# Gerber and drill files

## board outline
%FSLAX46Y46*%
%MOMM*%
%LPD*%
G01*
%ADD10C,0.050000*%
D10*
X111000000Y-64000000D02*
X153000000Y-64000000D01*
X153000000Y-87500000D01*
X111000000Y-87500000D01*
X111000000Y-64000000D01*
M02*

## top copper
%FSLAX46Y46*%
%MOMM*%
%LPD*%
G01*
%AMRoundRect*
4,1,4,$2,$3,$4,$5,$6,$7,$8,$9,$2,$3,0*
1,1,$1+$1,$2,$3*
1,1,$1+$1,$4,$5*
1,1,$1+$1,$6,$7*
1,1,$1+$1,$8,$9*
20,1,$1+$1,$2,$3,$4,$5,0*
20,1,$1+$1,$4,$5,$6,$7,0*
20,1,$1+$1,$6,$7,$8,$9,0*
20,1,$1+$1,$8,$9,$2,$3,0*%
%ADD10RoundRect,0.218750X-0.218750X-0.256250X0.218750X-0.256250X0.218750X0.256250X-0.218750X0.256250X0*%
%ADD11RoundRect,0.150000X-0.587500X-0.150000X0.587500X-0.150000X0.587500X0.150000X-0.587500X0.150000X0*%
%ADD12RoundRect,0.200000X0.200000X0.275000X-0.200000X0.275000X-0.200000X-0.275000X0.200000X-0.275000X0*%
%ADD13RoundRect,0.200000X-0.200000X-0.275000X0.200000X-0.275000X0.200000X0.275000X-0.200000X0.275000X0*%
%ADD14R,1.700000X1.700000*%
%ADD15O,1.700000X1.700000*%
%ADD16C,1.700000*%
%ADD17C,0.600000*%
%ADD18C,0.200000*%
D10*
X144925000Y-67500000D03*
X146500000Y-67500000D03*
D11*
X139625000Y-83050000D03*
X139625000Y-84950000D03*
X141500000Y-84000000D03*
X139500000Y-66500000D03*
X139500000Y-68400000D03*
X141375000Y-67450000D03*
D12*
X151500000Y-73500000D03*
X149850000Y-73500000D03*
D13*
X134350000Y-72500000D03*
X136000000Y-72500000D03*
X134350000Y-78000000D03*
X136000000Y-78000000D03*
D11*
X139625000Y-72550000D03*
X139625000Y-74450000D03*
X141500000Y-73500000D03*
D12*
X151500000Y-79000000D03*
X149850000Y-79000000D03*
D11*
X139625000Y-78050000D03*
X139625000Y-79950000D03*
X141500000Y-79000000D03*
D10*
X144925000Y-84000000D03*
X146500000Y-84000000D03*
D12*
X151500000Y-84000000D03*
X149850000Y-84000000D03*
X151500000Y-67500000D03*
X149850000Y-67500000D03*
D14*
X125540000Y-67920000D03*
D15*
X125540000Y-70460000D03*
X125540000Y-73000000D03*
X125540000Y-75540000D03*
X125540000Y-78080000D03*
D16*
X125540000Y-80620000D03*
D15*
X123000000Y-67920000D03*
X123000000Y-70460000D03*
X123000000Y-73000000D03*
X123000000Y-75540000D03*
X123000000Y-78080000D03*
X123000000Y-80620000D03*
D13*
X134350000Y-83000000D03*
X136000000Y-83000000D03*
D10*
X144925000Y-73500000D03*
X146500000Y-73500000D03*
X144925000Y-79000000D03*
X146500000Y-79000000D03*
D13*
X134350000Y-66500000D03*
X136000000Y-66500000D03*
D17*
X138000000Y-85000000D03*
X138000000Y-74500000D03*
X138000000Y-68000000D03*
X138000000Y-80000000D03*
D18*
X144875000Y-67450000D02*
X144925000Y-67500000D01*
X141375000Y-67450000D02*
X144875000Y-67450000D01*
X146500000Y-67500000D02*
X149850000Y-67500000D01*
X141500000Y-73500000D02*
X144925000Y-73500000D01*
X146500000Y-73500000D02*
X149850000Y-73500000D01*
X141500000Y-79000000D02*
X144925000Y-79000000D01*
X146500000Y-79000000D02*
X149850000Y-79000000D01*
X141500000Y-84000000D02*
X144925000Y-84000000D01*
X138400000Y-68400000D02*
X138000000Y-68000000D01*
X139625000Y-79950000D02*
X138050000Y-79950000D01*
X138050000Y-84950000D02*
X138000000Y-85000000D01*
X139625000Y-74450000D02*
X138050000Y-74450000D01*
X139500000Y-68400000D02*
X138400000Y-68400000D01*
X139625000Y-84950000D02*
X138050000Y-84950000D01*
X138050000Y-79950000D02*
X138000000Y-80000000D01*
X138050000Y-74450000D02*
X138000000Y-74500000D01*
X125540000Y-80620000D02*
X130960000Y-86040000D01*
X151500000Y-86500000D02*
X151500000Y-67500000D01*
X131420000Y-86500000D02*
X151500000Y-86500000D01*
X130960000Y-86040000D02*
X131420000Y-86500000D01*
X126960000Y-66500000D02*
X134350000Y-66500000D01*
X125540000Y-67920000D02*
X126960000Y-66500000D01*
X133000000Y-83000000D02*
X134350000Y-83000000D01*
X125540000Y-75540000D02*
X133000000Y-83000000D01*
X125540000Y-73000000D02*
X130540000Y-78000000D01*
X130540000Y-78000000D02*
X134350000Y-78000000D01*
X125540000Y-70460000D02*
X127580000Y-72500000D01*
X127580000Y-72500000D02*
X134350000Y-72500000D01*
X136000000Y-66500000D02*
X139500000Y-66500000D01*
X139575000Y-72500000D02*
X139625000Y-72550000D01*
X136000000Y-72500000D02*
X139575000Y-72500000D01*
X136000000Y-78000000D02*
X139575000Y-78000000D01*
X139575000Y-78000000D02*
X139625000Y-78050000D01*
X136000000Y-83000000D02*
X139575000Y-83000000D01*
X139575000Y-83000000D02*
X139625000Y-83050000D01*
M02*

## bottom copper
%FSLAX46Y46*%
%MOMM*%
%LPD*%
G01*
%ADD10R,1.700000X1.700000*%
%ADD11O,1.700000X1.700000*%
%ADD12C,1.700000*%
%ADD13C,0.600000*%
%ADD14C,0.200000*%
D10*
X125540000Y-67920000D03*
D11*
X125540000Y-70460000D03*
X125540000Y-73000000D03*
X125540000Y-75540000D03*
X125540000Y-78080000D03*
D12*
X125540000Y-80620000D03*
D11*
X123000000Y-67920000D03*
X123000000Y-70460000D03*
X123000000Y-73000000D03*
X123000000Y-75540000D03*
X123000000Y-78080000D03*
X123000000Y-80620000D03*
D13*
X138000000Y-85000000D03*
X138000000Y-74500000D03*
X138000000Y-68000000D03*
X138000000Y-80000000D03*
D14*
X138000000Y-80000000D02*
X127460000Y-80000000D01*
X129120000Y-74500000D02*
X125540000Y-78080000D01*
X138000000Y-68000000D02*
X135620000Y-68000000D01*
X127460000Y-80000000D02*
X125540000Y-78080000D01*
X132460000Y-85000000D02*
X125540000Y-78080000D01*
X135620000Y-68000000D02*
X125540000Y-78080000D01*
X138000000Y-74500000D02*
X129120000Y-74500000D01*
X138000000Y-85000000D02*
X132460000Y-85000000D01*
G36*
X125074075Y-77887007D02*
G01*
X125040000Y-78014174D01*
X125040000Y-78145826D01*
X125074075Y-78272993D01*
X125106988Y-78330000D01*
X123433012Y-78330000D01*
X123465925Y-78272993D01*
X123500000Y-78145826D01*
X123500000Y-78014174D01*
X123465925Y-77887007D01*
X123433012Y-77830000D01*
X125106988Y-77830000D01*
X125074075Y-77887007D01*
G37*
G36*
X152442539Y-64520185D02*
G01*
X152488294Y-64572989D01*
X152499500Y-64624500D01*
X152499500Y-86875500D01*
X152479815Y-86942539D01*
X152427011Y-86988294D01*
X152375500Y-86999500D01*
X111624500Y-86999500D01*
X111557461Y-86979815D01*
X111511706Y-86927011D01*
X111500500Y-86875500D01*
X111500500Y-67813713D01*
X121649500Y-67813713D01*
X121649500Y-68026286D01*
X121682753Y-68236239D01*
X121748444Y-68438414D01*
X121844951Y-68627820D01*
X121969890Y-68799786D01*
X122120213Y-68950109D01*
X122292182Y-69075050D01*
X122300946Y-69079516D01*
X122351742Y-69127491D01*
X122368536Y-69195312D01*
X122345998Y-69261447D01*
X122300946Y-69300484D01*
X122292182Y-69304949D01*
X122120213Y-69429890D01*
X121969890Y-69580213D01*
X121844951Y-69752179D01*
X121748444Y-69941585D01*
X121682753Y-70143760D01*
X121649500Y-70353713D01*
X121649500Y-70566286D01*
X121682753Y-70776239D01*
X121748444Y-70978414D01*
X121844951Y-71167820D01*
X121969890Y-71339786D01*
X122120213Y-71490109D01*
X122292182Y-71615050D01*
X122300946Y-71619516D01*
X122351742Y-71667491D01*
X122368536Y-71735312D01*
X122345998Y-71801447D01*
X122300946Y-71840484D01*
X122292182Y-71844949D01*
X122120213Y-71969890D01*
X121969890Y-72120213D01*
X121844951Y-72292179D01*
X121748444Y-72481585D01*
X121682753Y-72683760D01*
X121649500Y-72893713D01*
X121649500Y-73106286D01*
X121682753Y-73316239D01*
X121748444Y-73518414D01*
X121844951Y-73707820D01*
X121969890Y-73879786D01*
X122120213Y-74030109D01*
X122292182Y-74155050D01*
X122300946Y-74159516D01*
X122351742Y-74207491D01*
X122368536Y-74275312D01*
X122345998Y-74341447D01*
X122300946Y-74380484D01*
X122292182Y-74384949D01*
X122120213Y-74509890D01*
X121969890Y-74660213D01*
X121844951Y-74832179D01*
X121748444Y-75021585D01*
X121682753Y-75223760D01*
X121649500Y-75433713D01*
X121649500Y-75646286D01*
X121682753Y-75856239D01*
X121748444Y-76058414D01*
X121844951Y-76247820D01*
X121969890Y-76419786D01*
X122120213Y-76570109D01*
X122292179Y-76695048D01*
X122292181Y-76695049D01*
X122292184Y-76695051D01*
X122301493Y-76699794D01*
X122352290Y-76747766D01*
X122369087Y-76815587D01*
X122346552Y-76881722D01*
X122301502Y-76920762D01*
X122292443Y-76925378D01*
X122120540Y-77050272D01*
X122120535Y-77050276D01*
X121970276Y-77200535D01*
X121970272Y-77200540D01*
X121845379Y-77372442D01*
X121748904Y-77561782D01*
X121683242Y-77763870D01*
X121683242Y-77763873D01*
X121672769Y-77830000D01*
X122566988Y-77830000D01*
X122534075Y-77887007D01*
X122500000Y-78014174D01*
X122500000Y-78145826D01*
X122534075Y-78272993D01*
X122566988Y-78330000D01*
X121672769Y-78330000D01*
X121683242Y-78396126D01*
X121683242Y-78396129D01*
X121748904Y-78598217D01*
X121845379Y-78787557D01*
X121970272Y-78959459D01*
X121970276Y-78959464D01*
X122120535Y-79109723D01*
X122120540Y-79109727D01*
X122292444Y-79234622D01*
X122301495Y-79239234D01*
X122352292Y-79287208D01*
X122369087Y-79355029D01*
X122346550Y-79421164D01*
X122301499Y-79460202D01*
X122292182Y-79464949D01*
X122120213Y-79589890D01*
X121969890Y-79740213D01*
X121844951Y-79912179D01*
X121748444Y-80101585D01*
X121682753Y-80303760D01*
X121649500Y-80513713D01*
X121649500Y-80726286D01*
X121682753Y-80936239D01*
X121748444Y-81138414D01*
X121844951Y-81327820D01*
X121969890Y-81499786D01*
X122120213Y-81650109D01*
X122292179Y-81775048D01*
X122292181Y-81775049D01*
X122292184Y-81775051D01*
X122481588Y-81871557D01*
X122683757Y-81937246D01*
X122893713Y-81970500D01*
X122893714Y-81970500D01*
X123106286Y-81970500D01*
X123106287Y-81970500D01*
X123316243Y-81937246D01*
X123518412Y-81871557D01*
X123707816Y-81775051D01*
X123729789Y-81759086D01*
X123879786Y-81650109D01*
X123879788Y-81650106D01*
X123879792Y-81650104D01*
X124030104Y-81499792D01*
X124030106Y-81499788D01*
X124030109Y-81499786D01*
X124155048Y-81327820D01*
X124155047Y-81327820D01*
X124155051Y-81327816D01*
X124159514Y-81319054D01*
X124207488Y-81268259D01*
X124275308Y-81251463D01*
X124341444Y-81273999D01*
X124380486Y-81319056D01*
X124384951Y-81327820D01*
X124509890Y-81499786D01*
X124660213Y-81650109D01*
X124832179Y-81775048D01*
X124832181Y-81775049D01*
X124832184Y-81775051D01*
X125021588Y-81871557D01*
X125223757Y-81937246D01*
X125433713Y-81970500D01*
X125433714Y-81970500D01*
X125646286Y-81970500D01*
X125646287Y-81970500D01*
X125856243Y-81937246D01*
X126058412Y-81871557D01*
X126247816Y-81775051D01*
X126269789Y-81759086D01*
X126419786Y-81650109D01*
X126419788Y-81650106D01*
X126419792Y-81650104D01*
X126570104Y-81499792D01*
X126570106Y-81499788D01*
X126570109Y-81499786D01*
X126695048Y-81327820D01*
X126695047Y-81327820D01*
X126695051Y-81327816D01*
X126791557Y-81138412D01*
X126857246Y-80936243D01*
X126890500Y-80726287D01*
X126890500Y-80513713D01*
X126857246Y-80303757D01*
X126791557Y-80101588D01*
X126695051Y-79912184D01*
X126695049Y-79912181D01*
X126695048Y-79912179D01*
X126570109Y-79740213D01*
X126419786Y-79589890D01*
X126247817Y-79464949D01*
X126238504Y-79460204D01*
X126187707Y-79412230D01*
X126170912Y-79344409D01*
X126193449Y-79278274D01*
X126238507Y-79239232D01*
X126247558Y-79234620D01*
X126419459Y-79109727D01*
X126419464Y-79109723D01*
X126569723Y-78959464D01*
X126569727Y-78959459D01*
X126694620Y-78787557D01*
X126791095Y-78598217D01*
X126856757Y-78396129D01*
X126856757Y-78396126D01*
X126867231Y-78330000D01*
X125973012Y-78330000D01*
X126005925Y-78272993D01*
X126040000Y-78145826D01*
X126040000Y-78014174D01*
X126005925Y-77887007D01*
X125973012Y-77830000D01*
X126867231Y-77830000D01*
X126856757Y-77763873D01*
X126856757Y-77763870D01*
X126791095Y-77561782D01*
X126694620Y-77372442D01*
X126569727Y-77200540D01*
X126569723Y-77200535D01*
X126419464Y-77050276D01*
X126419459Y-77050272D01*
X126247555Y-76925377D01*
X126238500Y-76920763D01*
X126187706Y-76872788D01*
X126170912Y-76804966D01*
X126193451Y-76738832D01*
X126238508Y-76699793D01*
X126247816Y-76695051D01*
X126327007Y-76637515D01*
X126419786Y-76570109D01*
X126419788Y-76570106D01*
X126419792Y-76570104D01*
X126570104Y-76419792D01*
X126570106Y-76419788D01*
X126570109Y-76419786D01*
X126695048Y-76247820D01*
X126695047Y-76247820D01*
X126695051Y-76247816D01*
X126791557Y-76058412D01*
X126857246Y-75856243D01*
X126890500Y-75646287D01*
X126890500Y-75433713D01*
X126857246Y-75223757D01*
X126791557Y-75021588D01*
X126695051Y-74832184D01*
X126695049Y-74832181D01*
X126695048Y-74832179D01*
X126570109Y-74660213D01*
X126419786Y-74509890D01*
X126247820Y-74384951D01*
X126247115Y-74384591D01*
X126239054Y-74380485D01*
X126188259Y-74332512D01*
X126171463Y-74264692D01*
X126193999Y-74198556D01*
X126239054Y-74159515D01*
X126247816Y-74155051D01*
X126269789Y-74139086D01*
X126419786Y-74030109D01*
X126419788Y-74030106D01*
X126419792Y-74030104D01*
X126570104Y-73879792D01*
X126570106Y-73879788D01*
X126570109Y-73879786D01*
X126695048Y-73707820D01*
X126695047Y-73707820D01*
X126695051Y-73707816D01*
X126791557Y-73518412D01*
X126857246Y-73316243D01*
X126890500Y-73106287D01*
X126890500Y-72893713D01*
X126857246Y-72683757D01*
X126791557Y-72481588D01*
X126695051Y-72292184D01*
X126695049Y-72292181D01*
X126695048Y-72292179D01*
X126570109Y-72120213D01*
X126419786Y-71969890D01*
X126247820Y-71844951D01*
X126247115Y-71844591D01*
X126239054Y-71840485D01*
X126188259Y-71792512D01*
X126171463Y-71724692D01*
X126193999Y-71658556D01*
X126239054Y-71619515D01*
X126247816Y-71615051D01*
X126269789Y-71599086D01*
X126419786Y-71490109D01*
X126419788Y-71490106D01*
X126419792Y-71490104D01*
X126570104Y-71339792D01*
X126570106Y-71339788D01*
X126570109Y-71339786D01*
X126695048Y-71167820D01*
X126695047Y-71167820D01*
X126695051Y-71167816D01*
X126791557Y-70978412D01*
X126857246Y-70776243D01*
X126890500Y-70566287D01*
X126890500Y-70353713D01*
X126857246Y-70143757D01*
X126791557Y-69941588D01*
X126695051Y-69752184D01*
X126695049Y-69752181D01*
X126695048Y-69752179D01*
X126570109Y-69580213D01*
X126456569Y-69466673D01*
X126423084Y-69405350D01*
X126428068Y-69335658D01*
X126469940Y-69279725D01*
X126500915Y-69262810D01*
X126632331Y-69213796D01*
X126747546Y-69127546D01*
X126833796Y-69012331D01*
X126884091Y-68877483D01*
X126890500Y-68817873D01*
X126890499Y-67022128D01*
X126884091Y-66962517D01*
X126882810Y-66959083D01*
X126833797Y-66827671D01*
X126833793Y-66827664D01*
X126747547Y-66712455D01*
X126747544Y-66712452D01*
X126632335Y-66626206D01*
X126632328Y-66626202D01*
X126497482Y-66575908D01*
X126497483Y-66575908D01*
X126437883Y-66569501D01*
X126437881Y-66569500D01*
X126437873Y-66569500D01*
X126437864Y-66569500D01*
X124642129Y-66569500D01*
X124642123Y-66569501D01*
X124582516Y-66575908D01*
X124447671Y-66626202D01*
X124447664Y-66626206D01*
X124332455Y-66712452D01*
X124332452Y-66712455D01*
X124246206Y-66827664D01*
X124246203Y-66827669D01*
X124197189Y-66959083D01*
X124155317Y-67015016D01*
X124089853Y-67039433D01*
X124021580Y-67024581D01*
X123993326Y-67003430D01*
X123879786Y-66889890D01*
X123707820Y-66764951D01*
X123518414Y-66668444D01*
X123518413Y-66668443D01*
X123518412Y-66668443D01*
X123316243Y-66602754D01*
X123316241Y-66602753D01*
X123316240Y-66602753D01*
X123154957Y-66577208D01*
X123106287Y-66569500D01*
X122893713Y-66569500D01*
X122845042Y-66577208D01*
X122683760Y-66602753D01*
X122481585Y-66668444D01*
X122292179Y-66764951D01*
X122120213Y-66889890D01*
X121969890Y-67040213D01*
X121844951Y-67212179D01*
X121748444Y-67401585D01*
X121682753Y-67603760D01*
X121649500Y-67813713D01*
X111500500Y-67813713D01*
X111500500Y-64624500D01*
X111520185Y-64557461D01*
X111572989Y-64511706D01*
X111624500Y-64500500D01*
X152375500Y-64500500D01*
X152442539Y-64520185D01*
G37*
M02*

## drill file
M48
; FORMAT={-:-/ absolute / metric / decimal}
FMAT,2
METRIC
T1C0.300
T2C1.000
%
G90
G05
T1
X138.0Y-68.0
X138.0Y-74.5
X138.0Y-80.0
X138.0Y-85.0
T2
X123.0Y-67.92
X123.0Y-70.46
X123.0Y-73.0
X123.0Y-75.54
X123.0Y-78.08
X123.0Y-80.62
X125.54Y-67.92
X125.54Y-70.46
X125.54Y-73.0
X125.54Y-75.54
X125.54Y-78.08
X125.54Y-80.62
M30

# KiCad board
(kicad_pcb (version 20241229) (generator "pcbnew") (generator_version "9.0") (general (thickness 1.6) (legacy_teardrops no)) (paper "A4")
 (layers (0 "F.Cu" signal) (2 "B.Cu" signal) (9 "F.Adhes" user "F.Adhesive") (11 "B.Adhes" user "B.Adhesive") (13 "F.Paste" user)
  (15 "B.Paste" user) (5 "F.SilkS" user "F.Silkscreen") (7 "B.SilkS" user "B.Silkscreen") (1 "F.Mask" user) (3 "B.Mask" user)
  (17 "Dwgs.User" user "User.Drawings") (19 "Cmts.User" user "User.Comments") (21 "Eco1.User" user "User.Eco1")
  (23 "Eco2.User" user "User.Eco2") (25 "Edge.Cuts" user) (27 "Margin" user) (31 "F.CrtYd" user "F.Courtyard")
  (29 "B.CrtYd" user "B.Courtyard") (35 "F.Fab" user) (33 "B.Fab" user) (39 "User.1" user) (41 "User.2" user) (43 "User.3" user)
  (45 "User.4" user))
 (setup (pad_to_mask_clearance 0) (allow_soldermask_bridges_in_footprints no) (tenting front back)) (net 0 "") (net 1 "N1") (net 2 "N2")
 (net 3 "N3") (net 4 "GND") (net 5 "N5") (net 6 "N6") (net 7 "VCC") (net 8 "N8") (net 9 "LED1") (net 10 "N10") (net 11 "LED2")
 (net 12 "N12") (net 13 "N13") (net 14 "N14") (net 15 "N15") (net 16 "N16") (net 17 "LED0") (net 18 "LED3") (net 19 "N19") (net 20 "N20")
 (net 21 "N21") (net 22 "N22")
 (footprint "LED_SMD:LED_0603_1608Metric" (layer "F.Cu") (at 145.7125 67.5)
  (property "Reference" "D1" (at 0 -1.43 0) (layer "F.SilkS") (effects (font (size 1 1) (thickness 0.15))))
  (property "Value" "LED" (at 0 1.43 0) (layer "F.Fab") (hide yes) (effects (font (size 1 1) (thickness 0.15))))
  (pad "1" smd roundrect (at -0.7875 0) (size 0.875 0.95) (layers "F.Cu" "F.Mask" "F.Paste") (roundrect_rratio 0.25) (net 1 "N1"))
  (pad "2" smd roundrect (at 0.7875 0) (size 0.875 0.95) (layers "F.Cu" "F.Mask" "F.Paste") (roundrect_rratio 0.25) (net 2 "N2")))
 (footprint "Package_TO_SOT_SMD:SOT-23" (layer "F.Cu") (at 140.5625 84)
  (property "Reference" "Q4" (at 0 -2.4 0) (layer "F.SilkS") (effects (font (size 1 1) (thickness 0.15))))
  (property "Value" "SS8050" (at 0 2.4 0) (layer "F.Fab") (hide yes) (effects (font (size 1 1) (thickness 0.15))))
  (pad "1" smd roundrect (at -0.9375 -0.95) (size 1.475 0.6) (layers "F.Cu" "F.Mask" "F.Paste") (roundrect_rratio 0.25) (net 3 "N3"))
  (pad "2" smd roundrect (at -0.9375 0.95) (size 1.475 0.6) (layers "F.Cu" "F.Mask" "F.Paste") (roundrect_rratio 0.25) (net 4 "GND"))
  (pad "3" smd roundrect (at 0.9375 0) (size 1.475 0.6) (layers "F.Cu" "F.Mask" "F.Paste") (roundrect_rratio 0.25) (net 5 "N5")))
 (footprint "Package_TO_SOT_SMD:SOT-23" (layer "F.Cu") (at 140.4375 67.45)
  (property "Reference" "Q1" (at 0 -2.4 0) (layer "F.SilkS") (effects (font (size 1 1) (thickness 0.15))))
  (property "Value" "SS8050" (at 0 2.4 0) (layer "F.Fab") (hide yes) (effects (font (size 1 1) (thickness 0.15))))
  (pad "1" smd roundrect (at -0.9375 -0.95) (size 1.475 0.6) (layers "F.Cu" "F.Mask" "F.Paste") (roundrect_rratio 0.25) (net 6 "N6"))
  (pad "2" smd roundrect (at -0.9375 0.95) (size 1.475 0.6) (layers "F.Cu" "F.Mask" "F.Paste") (roundrect_rratio 0.25) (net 4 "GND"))
  (pad "3" smd roundrect (at 0.9375 0) (size 1.475 0.6) (layers "F.Cu" "F.Mask" "F.Paste") (roundrect_rratio 0.25) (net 1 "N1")))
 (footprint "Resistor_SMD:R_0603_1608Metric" (layer "F.Cu") (at 150.675 73.5 180)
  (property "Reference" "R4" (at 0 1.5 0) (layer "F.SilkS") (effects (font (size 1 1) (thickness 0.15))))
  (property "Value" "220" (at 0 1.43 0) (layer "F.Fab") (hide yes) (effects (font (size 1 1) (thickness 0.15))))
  (pad "1" smd roundrect (at -0.825 0 180) (size 0.8 0.95) (layers "F.Cu" "F.Mask" "F.Paste") (roundrect_rratio 0.25) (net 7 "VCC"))
  (pad "2" smd roundrect (at 0.825 0 180) (size 0.8 0.95) (layers "F.Cu" "F.Mask" "F.Paste") (roundrect_rratio 0.25) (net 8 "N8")))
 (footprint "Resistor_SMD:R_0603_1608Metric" (layer "F.Cu") (at 135.175 72.5)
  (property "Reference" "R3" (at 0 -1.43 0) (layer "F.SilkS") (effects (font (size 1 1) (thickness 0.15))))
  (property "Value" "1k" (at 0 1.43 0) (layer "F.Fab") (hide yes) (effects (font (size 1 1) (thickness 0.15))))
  (pad "1" smd roundrect (at -0.825 0) (size 0.8 0.95) (layers "F.Cu" "F.Mask" "F.Paste") (roundrect_rratio 0.25) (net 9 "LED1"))
  (pad "2" smd roundrect (at 0.825 0) (size 0.8 0.95) (layers "F.Cu" "F.Mask" "F.Paste") (roundrect_rratio 0.25) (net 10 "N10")))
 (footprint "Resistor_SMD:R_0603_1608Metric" (layer "F.Cu") (at 135.175 78)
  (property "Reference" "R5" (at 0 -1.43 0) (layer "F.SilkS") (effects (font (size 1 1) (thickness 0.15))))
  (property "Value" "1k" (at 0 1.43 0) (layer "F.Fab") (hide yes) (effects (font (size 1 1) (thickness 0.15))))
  (pad "1" smd roundrect (at -0.825 0) (size 0.8 0.95) (layers "F.Cu" "F.Mask" "F.Paste") (roundrect_rratio 0.25) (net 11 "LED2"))
  (pad "2" smd roundrect (at 0.825 0) (size 0.8 0.95) (layers "F.Cu" "F.Mask" "F.Paste") (roundrect_rratio 0.25) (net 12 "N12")))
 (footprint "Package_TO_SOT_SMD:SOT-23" (layer "F.Cu") (at 140.5625 73.5)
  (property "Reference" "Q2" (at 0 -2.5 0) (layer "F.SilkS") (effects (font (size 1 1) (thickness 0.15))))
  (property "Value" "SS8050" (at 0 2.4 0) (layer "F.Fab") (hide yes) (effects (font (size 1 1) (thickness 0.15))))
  (pad "1" smd roundrect (at -0.9375 -0.95) (size 1.475 0.6) (layers "F.Cu" "F.Mask" "F.Paste") (roundrect_rratio 0.25) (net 10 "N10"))
  (pad "2" smd roundrect (at -0.9375 0.95) (size 1.475 0.6) (layers "F.Cu" "F.Mask" "F.Paste") (roundrect_rratio 0.25) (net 4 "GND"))
  (pad "3" smd roundrect (at 0.9375 0) (size 1.475 0.6) (layers "F.Cu" "F.Mask" "F.Paste") (roundrect_rratio 0.25) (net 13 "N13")))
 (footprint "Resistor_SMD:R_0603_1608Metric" (layer "F.Cu") (at 150.675 79 180)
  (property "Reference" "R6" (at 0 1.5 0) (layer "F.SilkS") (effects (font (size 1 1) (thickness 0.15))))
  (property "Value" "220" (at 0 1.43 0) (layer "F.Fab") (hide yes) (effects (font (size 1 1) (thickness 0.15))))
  (pad "1" smd roundrect (at -0.825 0 180) (size 0.8 0.95) (layers "F.Cu" "F.Mask" "F.Paste") (roundrect_rratio 0.25) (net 7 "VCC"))
  (pad "2" smd roundrect (at 0.825 0 180) (size 0.8 0.95) (layers "F.Cu" "F.Mask" "F.Paste") (roundrect_rratio 0.25) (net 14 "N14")))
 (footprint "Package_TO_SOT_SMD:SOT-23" (layer "F.Cu") (at 140.5625 79)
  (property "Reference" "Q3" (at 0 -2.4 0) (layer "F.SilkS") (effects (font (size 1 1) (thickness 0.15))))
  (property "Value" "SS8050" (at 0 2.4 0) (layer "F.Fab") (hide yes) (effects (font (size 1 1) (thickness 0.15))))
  (pad "1" smd roundrect (at -0.9375 -0.95) (size 1.475 0.6) (layers "F.Cu" "F.Mask" "F.Paste") (roundrect_rratio 0.25) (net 12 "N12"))
  (pad "2" smd roundrect (at -0.9375 0.95) (size 1.475 0.6) (layers "F.Cu" "F.Mask" "F.Paste") (roundrect_rratio 0.25) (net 4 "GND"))
  (pad "3" smd roundrect (at 0.9375 0) (size 1.475 0.6) (layers "F.Cu" "F.Mask" "F.Paste") (roundrect_rratio 0.25) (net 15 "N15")))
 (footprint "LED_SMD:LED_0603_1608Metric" (layer "F.Cu") (at 145.7125 84)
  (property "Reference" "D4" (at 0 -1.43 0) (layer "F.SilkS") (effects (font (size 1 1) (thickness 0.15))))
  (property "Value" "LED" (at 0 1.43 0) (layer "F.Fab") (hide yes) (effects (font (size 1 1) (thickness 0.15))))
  (pad "1" smd roundrect (at -0.7875 0) (size 0.875 0.95) (layers "F.Cu" "F.Mask" "F.Paste") (roundrect_rratio 0.25) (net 5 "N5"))
  (pad "2" smd roundrect (at 0.7875 0) (size 0.875 0.95) (layers "F.Cu" "F.Mask" "F.Paste") (roundrect_rratio 0.25) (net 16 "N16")))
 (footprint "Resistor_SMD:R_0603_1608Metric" (layer "F.Cu") (at 150.675 84 180)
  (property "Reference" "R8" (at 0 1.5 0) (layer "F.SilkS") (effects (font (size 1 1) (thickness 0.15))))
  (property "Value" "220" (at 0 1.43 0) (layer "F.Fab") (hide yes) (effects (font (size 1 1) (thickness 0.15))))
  (pad "1" smd roundrect (at -0.825 0 180) (size 0.8 0.95) (layers "F.Cu" "F.Mask" "F.Paste") (roundrect_rratio 0.25) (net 7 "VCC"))
  (pad "2" smd roundrect (at 0.825 0 180) (size 0.8 0.95) (layers "F.Cu" "F.Mask" "F.Paste") (roundrect_rratio 0.25) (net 16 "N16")))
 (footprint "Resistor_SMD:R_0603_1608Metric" (layer "F.Cu") (at 150.675 67.5 180)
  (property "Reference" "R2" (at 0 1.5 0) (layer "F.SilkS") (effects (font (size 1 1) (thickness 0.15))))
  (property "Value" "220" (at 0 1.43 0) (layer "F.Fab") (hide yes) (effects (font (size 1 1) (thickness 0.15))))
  (pad "1" smd roundrect (at -0.825 0 180) (size 0.8 0.95) (layers "F.Cu" "F.Mask" "F.Paste") (roundrect_rratio 0.25) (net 7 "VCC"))
  (pad "2" smd roundrect (at 0.825 0 180) (size 0.8 0.95) (layers "F.Cu" "F.Mask" "F.Paste") (roundrect_rratio 0.25) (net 2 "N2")))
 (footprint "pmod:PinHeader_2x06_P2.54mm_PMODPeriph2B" (layer "F.Cu") (at 125.54 80.62 180)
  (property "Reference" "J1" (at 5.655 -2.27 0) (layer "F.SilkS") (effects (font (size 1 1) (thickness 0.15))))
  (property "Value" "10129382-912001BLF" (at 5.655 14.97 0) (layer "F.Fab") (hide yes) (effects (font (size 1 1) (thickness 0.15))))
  (pad "1" thru_hole rect (at 0 12.7 180) (size 1.7 1.7) (drill 1) (layers "*.Cu" "*.Mask") (remove_unused_layers no) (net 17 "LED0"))
  (pad "2" thru_hole oval (at 0 10.16 180) (size 1.7 1.7) (drill 1) (layers "*.Cu" "*.Mask") (remove_unused_layers no) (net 9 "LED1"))
  (pad "3" thru_hole oval (at 0 7.62 180) (size 1.7 1.7) (drill 1) (layers "*.Cu" "*.Mask") (remove_unused_layers no) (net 11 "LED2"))
  (pad "4" thru_hole oval (at 0 5.08 180) (size 1.7 1.7) (drill 1) (layers "*.Cu" "*.Mask") (remove_unused_layers no) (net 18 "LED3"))
  (pad "5" thru_hole oval (at 0 2.54 180) (size 1.7 1.7) (drill 1) (layers "*.Cu" "*.Mask") (remove_unused_layers no) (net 4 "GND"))
  (pad "6" thru_hole circle (at 0 0 180) (size 1.7 1.7) (drill 1) (layers "*.Cu" "*.Mask") (remove_unused_layers no) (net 7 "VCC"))
  (pad "7" thru_hole oval (at 2.54 12.7 180) (size 1.7 1.7) (drill 1) (layers "*.Cu" "*.Mask") (remove_unused_layers no) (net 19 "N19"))
  (pad "8" thru_hole oval (at 2.54 10.16 180) (size 1.7 1.7) (drill 1) (layers "*.Cu" "*.Mask") (remove_unused_layers no) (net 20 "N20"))
  (pad "9" thru_hole oval (at 2.54 7.62 180) (size 1.7 1.7) (drill 1) (layers "*.Cu" "*.Mask") (remove_unused_layers no) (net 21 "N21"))
  (pad "10" thru_hole oval (at 2.54 5.08 180) (size 1.7 1.7) (drill 1) (layers "*.Cu" "*.Mask") (remove_unused_layers no) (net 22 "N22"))
  (pad "11" thru_hole oval (at 2.54 2.54 180) (size 1.7 1.7) (drill 1) (layers "*.Cu" "*.Mask") (remove_unused_layers no) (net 4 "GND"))
  (pad "12" thru_hole oval (at 2.54 0 180) (size 1.7 1.7) (drill 1) (layers "*.Cu" "*.Mask") (remove_unused_layers no) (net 7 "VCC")))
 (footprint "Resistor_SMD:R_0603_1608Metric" (layer "F.Cu") (at 135.175 83)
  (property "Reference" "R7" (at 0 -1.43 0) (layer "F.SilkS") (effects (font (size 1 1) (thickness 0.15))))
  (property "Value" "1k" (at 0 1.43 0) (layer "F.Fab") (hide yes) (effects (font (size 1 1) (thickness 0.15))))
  (pad "1" smd roundrect (at -0.825 0) (size 0.8 0.95) (layers "F.Cu" "F.Mask" "F.Paste") (roundrect_rratio 0.25) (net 18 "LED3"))
  (pad "2" smd roundrect (at 0.825 0) (size 0.8 0.95) (layers "F.Cu" "F.Mask" "F.Paste") (roundrect_rratio 0.25) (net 3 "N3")))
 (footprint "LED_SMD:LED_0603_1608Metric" (layer "F.Cu") (at 145.7125 73.5)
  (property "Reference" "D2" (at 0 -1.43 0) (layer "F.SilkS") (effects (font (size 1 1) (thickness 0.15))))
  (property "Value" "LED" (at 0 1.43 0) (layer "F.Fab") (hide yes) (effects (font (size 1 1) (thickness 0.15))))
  (pad "1" smd roundrect (at -0.7875 0) (size 0.875 0.95) (layers "F.Cu" "F.Mask" "F.Paste") (roundrect_rratio 0.25) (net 13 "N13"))
  (pad "2" smd roundrect (at 0.7875 0) (size 0.875 0.95) (layers "F.Cu" "F.Mask" "F.Paste") (roundrect_rratio 0.25) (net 8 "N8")))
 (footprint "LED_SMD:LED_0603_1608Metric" (layer "F.Cu") (at 145.7125 79)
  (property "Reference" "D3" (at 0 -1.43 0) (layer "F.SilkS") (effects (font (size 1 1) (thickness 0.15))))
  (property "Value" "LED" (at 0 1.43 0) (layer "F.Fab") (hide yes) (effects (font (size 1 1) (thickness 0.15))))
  (pad "1" smd roundrect (at -0.7875 0) (size 0.875 0.95) (layers "F.Cu" "F.Mask" "F.Paste") (roundrect_rratio 0.25) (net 15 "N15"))
  (pad "2" smd roundrect (at 0.7875 0) (size 0.875 0.95) (layers "F.Cu" "F.Mask" "F.Paste") (roundrect_rratio 0.25) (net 14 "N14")))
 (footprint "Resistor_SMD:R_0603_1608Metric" (layer "F.Cu") (at 135.175 66.5)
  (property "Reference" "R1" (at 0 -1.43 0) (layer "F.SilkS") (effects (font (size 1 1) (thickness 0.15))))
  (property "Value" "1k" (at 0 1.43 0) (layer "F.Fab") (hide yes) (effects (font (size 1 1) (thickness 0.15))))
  (pad "1" smd roundrect (at -0.825 0) (size 0.8 0.95) (layers "F.Cu" "F.Mask" "F.Paste") (roundrect_rratio 0.25) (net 17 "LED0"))
  (pad "2" smd roundrect (at 0.825 0) (size 0.8 0.95) (layers "F.Cu" "F.Mask" "F.Paste") (roundrect_rratio 0.25) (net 6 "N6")))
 (gr_rect (start 111 64) (end 153 87.5) (stroke (width 0.05) (type default)) (fill no) (layer "Edge.Cuts"))
 (segment (start 144.875 67.45) (end 144.925 67.5) (width 0.2) (layer "F.Cu") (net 1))
 (segment (start 141.375 67.45) (end 144.875 67.45) (width 0.2) (layer "F.Cu") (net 1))
 (segment (start 146.5 67.5) (end 149.85 67.5) (width 0.2) (layer "F.Cu") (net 2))
 (segment (start 141.5 73.5) (end 144.925 73.5) (width 0.2) (layer "F.Cu") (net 13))
 (segment (start 146.5 73.5) (end 149.85 73.5) (width 0.2) (layer "F.Cu") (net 8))
 (segment (start 141.5 79) (end 144.925 79) (width 0.2) (layer "F.Cu") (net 15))
 (segment (start 146.5 79) (end 149.85 79) (width 0.2) (layer "F.Cu") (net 14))
 (segment (start 141.5 84) (end 144.925 84) (width 0.2) (layer "F.Cu") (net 5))
 (segment (start 138.4 68.4) (end 138 68) (width 0.2) (layer "F.Cu") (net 4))
 (segment (start 139.625 79.95) (end 138.05 79.95) (width 0.2) (layer "F.Cu") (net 4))
 (segment (start 138.05 84.95) (end 138 85) (width 0.2) (layer "F.Cu") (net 4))
 (segment (start 139.625 74.45) (end 138.05 74.45) (width 0.2) (layer "F.Cu") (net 4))
 (segment (start 139.5 68.4) (end 138.4 68.4) (width 0.2) (layer "F.Cu") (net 4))
 (segment (start 139.625 84.95) (end 138.05 84.95) (width 0.2) (layer "F.Cu") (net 4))
 (segment (start 138.05 79.95) (end 138 80) (width 0.2) (layer "F.Cu") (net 4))
 (segment (start 138.05 74.45) (end 138 74.5) (width 0.2) (layer "F.Cu") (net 4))
 (via (at 138 85) (size 0.6) (drill 0.3) (layers "F.Cu" "B.Cu") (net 4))
 (via (at 138 74.5) (size 0.6) (drill 0.3) (layers "F.Cu" "B.Cu") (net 4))
 (via (at 138 68) (size 0.6) (drill 0.3) (layers "F.Cu" "B.Cu") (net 4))
 (via (at 138 80) (size 0.6) (drill 0.3) (layers "F.Cu" "B.Cu") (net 4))
 (segment (start 138 80) (end 127.46 80) (width 0.2) (layer "B.Cu") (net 4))
 (segment (start 129.12 74.5) (end 125.54 78.08) (width 0.2) (layer "B.Cu") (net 4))
 (segment (start 138 68) (end 135.62 68) (width 0.2) (layer "B.Cu") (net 4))
 (segment (start 127.46 80) (end 125.54 78.08) (width 0.2) (layer "B.Cu") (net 4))
 (segment (start 132.46 85) (end 125.54 78.08) (width 0.2) (layer "B.Cu") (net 4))
 (segment (start 135.62 68) (end 125.54 78.08) (width 0.2) (layer "B.Cu") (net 4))
 (segment (start 138 74.5) (end 129.12 74.5) (width 0.2) (layer "B.Cu") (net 4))
 (segment (start 138 85) (end 132.46 85) (width 0.2) (layer "B.Cu") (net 4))
 (segment (start 125.54 80.62) (end 130.96 86.04) (width 0.2) (layer "F.Cu") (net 7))
 (segment (start 151.5 86.5) (end 151.5 67.5) (width 0.2) (layer "F.Cu") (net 7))
 (segment (start 131.42 86.5) (end 151.5 86.5) (width 0.2) (layer "F.Cu") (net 7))
 (segment (start 130.96 86.04) (end 131.42 86.5) (width 0.2) (layer "F.Cu") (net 7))
 (segment (start 126.96 66.5) (end 134.35 66.5) (width 0.2) (layer "F.Cu") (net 17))
 (segment (start 125.54 67.92) (end 126.96 66.5) (width 0.2) (layer "F.Cu") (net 17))
 (segment (start 133 83) (end 134.35 83) (width 0.2) (layer "F.Cu") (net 18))
 (segment (start 125.54 75.54) (end 133 83) (width 0.2) (layer "F.Cu") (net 18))
 (segment (start 125.54 73) (end 130.54 78) (width 0.2) (layer "F.Cu") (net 11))
 (segment (start 130.54 78) (end 134.35 78) (width 0.2) (layer "F.Cu") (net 11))
 (segment (start 125.54 70.46) (end 127.58 72.5) (width 0.2) (layer "F.Cu") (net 9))
 (segment (start 127.58 72.5) (end 134.35 72.5) (width 0.2) (layer "F.Cu") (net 9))
 (segment (start 136 66.5) (end 139.5 66.5) (width 0.2) (layer "F.Cu") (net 6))
 (segment (start 139.575 72.5) (end 139.625 72.55) (width 0.2) (layer "F.Cu") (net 10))
 (segment (start 136 72.5) (end 139.575 72.5) (width 0.2) (layer "F.Cu") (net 10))
 (segment (start 136 78) (end 139.575 78) (width 0.2) (layer "F.Cu") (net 12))
 (segment (start 139.575 78) (end 139.625 78.05) (width 0.2) (layer "F.Cu") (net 12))
 (segment (start 136 83) (end 139.575 83) (width 0.2) (layer "F.Cu") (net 3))
 (segment (start 139.575 83) (end 139.625 83.05) (width 0.2) (layer "F.Cu") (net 3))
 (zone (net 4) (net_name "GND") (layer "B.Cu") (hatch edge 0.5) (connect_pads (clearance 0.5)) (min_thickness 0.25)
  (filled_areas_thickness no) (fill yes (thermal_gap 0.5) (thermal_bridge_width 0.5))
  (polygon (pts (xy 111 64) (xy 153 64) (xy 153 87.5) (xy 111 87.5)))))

